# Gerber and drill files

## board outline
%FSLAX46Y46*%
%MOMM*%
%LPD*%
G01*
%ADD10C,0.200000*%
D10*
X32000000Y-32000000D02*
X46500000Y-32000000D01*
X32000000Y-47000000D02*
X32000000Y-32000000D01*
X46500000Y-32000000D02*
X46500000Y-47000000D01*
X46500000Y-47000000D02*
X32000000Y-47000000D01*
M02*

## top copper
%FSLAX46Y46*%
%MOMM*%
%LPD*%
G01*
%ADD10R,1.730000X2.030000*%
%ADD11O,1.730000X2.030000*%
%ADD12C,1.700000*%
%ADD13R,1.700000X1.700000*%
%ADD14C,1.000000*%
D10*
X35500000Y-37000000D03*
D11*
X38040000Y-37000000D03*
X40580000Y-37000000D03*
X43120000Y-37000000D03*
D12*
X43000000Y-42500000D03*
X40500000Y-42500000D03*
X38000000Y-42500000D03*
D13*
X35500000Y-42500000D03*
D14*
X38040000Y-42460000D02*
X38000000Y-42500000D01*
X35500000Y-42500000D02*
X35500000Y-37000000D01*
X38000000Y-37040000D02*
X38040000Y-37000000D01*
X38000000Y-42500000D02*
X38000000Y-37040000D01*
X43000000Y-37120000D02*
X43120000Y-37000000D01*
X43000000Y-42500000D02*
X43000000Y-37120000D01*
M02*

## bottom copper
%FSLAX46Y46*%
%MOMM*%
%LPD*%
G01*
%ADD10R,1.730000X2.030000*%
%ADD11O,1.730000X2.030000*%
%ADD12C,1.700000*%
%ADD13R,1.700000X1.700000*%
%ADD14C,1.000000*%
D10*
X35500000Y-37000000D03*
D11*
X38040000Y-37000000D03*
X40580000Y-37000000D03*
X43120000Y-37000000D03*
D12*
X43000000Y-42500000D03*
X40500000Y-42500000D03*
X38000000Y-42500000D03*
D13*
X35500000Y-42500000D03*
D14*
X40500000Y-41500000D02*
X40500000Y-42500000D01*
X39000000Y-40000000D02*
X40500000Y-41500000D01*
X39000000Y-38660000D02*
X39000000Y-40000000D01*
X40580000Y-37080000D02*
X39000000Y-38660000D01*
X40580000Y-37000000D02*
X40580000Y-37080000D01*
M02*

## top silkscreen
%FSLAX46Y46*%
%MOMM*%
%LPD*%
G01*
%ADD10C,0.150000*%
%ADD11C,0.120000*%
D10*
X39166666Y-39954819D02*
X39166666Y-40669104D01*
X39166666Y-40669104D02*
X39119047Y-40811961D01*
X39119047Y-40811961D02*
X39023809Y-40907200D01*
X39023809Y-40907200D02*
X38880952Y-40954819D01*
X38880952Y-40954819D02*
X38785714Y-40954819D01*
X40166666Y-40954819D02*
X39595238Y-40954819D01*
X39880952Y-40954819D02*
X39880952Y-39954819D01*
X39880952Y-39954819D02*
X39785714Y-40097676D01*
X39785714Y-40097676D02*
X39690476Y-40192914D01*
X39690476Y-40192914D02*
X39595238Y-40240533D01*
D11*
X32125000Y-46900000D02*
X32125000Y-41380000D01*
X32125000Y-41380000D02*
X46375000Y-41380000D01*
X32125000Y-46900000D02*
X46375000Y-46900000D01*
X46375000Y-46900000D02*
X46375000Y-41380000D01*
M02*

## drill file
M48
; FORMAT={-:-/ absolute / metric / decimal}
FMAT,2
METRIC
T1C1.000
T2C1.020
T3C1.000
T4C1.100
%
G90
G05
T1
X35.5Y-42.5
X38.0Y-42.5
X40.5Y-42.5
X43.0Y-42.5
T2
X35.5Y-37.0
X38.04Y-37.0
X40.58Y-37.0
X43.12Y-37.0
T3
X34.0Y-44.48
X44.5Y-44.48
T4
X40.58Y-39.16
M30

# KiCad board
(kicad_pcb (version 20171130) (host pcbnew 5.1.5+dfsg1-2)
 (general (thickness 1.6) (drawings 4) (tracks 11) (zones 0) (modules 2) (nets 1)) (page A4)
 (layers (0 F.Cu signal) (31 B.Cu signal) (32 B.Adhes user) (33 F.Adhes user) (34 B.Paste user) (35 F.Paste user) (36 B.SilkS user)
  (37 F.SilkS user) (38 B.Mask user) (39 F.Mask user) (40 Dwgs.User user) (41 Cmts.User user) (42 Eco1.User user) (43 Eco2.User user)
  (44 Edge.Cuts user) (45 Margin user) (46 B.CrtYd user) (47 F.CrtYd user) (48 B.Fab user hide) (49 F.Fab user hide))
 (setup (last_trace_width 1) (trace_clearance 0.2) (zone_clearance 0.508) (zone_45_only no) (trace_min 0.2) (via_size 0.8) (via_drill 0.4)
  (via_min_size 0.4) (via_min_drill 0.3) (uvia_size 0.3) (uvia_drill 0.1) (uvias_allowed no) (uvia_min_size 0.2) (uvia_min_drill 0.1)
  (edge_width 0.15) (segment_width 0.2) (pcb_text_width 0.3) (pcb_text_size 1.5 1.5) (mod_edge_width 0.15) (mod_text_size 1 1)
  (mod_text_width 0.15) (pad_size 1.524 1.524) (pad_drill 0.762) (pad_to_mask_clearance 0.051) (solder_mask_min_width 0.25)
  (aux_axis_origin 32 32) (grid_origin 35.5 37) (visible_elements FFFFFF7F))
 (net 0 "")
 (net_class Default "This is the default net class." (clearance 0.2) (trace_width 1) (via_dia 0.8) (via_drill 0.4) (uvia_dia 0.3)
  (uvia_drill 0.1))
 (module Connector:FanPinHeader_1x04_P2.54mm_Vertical (layer B.Cu) (at 35.5 37)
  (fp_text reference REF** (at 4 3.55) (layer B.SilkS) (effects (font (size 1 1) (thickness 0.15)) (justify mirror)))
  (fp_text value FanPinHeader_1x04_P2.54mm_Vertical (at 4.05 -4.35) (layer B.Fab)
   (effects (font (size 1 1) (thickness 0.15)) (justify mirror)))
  (pad 1 thru_hole rect (at 0 0 270) (size 2.03 1.73) (drill 1.02) (layers *.Cu *.Mask))
  (pad 2 thru_hole oval (at 2.54 0 270) (size 2.03 1.73) (drill 1.02) (layers *.Cu *.Mask))
  (pad 3 thru_hole oval (at 5.08 0 270) (size 2.03 1.73) (drill 1.02) (layers *.Cu *.Mask))
  (pad 4 thru_hole oval (at 7.62 0 270) (size 2.03 1.73) (drill 1.02) (layers *.Cu *.Mask))
  (pad "" np_thru_hole circle (at 5.08 2.16 270) (size 1.1 1.1) (drill 1.1) (layers *.Cu *.Mask)))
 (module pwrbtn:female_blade (layer F.Cu) (at 39.25 42.5)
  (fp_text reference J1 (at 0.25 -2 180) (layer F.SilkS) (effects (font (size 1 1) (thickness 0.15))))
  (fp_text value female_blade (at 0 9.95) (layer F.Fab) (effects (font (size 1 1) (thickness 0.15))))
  (fp_line (start -7.125 4.4) (end -7.125 -1.12) (layer F.SilkS) (width 0.12))
  (fp_line (start -7.125 -1.12) (end 7.125 -1.12) (layer F.SilkS) (width 0.12))
  (fp_line (start -7.125 4.4) (end 7.125 4.4) (layer F.SilkS) (width 0.12))
  (fp_line (start 7.125 4.4) (end 7.125 -1.12) (layer F.SilkS) (width 0.12))
  (pad 4 thru_hole circle (at 3.75 0 90) (size 1.7 1.7) (drill 1) (layers *.Cu *.Mask))
  (pad 3 thru_hole circle (at 1.25 0 90) (size 1.7 1.7) (drill 1) (layers *.Cu *.Mask))
  (pad 2 thru_hole circle (at -1.25 0 90) (size 1.7 1.7) (drill 1) (layers *.Cu *.Mask))
  (pad 1 thru_hole rect (at -3.75 0 90) (size 1.7 1.7) (drill 1) (layers *.Cu *.Mask))
  (pad "" np_thru_hole circle (at 5.25 1.98 90) (size 1 1) (drill 1) (layers *.Cu *.Mask))
  (pad "" np_thru_hole circle (at -5.25 1.98 90) (size 1 1) (drill 1) (layers *.Cu *.Mask)))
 (gr_line (start 32 32) (end 46.5 32) (layer Edge.Cuts) (width 0.2))
 (gr_line (start 32 47) (end 32 32) (layer Edge.Cuts) (width 0.2))
 (gr_line (start 46.5 32) (end 46.5 47) (layer Edge.Cuts) (width 0.2))
 (gr_line (start 46.5 47) (end 32 47) (layer Edge.Cuts) (width 0.2))
 (segment (start 38.04 42.46) (end 38 42.5) (width 1) (layer F.Cu) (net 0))
 (segment (start 35.5 42.5) (end 35.5 37) (width 1) (layer F.Cu) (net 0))
 (segment (start 38 37.04) (end 38.04 37) (width 1) (layer F.Cu) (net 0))
 (segment (start 38 42.5) (end 38 37.04) (width 1) (layer F.Cu) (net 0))
 (segment (start 43 37.12) (end 43.12 37) (width 1) (layer F.Cu) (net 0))
 (segment (start 43 42.5) (end 43 37.12) (width 1) (layer F.Cu) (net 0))
 (segment (start 40.5 41.5) (end 40.5 42.5) (width 1) (layer B.Cu) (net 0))
 (segment (start 39 40) (end 40.5 41.5) (width 1) (layer B.Cu) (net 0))
 (segment (start 39 38.66) (end 39 40) (width 1) (layer B.Cu) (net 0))
 (segment (start 40.58 37.08) (end 39 38.66) (width 1) (layer B.Cu) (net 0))
 (segment (start 40.58 37) (end 40.58 37.08) (width 1) (layer B.Cu) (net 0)))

